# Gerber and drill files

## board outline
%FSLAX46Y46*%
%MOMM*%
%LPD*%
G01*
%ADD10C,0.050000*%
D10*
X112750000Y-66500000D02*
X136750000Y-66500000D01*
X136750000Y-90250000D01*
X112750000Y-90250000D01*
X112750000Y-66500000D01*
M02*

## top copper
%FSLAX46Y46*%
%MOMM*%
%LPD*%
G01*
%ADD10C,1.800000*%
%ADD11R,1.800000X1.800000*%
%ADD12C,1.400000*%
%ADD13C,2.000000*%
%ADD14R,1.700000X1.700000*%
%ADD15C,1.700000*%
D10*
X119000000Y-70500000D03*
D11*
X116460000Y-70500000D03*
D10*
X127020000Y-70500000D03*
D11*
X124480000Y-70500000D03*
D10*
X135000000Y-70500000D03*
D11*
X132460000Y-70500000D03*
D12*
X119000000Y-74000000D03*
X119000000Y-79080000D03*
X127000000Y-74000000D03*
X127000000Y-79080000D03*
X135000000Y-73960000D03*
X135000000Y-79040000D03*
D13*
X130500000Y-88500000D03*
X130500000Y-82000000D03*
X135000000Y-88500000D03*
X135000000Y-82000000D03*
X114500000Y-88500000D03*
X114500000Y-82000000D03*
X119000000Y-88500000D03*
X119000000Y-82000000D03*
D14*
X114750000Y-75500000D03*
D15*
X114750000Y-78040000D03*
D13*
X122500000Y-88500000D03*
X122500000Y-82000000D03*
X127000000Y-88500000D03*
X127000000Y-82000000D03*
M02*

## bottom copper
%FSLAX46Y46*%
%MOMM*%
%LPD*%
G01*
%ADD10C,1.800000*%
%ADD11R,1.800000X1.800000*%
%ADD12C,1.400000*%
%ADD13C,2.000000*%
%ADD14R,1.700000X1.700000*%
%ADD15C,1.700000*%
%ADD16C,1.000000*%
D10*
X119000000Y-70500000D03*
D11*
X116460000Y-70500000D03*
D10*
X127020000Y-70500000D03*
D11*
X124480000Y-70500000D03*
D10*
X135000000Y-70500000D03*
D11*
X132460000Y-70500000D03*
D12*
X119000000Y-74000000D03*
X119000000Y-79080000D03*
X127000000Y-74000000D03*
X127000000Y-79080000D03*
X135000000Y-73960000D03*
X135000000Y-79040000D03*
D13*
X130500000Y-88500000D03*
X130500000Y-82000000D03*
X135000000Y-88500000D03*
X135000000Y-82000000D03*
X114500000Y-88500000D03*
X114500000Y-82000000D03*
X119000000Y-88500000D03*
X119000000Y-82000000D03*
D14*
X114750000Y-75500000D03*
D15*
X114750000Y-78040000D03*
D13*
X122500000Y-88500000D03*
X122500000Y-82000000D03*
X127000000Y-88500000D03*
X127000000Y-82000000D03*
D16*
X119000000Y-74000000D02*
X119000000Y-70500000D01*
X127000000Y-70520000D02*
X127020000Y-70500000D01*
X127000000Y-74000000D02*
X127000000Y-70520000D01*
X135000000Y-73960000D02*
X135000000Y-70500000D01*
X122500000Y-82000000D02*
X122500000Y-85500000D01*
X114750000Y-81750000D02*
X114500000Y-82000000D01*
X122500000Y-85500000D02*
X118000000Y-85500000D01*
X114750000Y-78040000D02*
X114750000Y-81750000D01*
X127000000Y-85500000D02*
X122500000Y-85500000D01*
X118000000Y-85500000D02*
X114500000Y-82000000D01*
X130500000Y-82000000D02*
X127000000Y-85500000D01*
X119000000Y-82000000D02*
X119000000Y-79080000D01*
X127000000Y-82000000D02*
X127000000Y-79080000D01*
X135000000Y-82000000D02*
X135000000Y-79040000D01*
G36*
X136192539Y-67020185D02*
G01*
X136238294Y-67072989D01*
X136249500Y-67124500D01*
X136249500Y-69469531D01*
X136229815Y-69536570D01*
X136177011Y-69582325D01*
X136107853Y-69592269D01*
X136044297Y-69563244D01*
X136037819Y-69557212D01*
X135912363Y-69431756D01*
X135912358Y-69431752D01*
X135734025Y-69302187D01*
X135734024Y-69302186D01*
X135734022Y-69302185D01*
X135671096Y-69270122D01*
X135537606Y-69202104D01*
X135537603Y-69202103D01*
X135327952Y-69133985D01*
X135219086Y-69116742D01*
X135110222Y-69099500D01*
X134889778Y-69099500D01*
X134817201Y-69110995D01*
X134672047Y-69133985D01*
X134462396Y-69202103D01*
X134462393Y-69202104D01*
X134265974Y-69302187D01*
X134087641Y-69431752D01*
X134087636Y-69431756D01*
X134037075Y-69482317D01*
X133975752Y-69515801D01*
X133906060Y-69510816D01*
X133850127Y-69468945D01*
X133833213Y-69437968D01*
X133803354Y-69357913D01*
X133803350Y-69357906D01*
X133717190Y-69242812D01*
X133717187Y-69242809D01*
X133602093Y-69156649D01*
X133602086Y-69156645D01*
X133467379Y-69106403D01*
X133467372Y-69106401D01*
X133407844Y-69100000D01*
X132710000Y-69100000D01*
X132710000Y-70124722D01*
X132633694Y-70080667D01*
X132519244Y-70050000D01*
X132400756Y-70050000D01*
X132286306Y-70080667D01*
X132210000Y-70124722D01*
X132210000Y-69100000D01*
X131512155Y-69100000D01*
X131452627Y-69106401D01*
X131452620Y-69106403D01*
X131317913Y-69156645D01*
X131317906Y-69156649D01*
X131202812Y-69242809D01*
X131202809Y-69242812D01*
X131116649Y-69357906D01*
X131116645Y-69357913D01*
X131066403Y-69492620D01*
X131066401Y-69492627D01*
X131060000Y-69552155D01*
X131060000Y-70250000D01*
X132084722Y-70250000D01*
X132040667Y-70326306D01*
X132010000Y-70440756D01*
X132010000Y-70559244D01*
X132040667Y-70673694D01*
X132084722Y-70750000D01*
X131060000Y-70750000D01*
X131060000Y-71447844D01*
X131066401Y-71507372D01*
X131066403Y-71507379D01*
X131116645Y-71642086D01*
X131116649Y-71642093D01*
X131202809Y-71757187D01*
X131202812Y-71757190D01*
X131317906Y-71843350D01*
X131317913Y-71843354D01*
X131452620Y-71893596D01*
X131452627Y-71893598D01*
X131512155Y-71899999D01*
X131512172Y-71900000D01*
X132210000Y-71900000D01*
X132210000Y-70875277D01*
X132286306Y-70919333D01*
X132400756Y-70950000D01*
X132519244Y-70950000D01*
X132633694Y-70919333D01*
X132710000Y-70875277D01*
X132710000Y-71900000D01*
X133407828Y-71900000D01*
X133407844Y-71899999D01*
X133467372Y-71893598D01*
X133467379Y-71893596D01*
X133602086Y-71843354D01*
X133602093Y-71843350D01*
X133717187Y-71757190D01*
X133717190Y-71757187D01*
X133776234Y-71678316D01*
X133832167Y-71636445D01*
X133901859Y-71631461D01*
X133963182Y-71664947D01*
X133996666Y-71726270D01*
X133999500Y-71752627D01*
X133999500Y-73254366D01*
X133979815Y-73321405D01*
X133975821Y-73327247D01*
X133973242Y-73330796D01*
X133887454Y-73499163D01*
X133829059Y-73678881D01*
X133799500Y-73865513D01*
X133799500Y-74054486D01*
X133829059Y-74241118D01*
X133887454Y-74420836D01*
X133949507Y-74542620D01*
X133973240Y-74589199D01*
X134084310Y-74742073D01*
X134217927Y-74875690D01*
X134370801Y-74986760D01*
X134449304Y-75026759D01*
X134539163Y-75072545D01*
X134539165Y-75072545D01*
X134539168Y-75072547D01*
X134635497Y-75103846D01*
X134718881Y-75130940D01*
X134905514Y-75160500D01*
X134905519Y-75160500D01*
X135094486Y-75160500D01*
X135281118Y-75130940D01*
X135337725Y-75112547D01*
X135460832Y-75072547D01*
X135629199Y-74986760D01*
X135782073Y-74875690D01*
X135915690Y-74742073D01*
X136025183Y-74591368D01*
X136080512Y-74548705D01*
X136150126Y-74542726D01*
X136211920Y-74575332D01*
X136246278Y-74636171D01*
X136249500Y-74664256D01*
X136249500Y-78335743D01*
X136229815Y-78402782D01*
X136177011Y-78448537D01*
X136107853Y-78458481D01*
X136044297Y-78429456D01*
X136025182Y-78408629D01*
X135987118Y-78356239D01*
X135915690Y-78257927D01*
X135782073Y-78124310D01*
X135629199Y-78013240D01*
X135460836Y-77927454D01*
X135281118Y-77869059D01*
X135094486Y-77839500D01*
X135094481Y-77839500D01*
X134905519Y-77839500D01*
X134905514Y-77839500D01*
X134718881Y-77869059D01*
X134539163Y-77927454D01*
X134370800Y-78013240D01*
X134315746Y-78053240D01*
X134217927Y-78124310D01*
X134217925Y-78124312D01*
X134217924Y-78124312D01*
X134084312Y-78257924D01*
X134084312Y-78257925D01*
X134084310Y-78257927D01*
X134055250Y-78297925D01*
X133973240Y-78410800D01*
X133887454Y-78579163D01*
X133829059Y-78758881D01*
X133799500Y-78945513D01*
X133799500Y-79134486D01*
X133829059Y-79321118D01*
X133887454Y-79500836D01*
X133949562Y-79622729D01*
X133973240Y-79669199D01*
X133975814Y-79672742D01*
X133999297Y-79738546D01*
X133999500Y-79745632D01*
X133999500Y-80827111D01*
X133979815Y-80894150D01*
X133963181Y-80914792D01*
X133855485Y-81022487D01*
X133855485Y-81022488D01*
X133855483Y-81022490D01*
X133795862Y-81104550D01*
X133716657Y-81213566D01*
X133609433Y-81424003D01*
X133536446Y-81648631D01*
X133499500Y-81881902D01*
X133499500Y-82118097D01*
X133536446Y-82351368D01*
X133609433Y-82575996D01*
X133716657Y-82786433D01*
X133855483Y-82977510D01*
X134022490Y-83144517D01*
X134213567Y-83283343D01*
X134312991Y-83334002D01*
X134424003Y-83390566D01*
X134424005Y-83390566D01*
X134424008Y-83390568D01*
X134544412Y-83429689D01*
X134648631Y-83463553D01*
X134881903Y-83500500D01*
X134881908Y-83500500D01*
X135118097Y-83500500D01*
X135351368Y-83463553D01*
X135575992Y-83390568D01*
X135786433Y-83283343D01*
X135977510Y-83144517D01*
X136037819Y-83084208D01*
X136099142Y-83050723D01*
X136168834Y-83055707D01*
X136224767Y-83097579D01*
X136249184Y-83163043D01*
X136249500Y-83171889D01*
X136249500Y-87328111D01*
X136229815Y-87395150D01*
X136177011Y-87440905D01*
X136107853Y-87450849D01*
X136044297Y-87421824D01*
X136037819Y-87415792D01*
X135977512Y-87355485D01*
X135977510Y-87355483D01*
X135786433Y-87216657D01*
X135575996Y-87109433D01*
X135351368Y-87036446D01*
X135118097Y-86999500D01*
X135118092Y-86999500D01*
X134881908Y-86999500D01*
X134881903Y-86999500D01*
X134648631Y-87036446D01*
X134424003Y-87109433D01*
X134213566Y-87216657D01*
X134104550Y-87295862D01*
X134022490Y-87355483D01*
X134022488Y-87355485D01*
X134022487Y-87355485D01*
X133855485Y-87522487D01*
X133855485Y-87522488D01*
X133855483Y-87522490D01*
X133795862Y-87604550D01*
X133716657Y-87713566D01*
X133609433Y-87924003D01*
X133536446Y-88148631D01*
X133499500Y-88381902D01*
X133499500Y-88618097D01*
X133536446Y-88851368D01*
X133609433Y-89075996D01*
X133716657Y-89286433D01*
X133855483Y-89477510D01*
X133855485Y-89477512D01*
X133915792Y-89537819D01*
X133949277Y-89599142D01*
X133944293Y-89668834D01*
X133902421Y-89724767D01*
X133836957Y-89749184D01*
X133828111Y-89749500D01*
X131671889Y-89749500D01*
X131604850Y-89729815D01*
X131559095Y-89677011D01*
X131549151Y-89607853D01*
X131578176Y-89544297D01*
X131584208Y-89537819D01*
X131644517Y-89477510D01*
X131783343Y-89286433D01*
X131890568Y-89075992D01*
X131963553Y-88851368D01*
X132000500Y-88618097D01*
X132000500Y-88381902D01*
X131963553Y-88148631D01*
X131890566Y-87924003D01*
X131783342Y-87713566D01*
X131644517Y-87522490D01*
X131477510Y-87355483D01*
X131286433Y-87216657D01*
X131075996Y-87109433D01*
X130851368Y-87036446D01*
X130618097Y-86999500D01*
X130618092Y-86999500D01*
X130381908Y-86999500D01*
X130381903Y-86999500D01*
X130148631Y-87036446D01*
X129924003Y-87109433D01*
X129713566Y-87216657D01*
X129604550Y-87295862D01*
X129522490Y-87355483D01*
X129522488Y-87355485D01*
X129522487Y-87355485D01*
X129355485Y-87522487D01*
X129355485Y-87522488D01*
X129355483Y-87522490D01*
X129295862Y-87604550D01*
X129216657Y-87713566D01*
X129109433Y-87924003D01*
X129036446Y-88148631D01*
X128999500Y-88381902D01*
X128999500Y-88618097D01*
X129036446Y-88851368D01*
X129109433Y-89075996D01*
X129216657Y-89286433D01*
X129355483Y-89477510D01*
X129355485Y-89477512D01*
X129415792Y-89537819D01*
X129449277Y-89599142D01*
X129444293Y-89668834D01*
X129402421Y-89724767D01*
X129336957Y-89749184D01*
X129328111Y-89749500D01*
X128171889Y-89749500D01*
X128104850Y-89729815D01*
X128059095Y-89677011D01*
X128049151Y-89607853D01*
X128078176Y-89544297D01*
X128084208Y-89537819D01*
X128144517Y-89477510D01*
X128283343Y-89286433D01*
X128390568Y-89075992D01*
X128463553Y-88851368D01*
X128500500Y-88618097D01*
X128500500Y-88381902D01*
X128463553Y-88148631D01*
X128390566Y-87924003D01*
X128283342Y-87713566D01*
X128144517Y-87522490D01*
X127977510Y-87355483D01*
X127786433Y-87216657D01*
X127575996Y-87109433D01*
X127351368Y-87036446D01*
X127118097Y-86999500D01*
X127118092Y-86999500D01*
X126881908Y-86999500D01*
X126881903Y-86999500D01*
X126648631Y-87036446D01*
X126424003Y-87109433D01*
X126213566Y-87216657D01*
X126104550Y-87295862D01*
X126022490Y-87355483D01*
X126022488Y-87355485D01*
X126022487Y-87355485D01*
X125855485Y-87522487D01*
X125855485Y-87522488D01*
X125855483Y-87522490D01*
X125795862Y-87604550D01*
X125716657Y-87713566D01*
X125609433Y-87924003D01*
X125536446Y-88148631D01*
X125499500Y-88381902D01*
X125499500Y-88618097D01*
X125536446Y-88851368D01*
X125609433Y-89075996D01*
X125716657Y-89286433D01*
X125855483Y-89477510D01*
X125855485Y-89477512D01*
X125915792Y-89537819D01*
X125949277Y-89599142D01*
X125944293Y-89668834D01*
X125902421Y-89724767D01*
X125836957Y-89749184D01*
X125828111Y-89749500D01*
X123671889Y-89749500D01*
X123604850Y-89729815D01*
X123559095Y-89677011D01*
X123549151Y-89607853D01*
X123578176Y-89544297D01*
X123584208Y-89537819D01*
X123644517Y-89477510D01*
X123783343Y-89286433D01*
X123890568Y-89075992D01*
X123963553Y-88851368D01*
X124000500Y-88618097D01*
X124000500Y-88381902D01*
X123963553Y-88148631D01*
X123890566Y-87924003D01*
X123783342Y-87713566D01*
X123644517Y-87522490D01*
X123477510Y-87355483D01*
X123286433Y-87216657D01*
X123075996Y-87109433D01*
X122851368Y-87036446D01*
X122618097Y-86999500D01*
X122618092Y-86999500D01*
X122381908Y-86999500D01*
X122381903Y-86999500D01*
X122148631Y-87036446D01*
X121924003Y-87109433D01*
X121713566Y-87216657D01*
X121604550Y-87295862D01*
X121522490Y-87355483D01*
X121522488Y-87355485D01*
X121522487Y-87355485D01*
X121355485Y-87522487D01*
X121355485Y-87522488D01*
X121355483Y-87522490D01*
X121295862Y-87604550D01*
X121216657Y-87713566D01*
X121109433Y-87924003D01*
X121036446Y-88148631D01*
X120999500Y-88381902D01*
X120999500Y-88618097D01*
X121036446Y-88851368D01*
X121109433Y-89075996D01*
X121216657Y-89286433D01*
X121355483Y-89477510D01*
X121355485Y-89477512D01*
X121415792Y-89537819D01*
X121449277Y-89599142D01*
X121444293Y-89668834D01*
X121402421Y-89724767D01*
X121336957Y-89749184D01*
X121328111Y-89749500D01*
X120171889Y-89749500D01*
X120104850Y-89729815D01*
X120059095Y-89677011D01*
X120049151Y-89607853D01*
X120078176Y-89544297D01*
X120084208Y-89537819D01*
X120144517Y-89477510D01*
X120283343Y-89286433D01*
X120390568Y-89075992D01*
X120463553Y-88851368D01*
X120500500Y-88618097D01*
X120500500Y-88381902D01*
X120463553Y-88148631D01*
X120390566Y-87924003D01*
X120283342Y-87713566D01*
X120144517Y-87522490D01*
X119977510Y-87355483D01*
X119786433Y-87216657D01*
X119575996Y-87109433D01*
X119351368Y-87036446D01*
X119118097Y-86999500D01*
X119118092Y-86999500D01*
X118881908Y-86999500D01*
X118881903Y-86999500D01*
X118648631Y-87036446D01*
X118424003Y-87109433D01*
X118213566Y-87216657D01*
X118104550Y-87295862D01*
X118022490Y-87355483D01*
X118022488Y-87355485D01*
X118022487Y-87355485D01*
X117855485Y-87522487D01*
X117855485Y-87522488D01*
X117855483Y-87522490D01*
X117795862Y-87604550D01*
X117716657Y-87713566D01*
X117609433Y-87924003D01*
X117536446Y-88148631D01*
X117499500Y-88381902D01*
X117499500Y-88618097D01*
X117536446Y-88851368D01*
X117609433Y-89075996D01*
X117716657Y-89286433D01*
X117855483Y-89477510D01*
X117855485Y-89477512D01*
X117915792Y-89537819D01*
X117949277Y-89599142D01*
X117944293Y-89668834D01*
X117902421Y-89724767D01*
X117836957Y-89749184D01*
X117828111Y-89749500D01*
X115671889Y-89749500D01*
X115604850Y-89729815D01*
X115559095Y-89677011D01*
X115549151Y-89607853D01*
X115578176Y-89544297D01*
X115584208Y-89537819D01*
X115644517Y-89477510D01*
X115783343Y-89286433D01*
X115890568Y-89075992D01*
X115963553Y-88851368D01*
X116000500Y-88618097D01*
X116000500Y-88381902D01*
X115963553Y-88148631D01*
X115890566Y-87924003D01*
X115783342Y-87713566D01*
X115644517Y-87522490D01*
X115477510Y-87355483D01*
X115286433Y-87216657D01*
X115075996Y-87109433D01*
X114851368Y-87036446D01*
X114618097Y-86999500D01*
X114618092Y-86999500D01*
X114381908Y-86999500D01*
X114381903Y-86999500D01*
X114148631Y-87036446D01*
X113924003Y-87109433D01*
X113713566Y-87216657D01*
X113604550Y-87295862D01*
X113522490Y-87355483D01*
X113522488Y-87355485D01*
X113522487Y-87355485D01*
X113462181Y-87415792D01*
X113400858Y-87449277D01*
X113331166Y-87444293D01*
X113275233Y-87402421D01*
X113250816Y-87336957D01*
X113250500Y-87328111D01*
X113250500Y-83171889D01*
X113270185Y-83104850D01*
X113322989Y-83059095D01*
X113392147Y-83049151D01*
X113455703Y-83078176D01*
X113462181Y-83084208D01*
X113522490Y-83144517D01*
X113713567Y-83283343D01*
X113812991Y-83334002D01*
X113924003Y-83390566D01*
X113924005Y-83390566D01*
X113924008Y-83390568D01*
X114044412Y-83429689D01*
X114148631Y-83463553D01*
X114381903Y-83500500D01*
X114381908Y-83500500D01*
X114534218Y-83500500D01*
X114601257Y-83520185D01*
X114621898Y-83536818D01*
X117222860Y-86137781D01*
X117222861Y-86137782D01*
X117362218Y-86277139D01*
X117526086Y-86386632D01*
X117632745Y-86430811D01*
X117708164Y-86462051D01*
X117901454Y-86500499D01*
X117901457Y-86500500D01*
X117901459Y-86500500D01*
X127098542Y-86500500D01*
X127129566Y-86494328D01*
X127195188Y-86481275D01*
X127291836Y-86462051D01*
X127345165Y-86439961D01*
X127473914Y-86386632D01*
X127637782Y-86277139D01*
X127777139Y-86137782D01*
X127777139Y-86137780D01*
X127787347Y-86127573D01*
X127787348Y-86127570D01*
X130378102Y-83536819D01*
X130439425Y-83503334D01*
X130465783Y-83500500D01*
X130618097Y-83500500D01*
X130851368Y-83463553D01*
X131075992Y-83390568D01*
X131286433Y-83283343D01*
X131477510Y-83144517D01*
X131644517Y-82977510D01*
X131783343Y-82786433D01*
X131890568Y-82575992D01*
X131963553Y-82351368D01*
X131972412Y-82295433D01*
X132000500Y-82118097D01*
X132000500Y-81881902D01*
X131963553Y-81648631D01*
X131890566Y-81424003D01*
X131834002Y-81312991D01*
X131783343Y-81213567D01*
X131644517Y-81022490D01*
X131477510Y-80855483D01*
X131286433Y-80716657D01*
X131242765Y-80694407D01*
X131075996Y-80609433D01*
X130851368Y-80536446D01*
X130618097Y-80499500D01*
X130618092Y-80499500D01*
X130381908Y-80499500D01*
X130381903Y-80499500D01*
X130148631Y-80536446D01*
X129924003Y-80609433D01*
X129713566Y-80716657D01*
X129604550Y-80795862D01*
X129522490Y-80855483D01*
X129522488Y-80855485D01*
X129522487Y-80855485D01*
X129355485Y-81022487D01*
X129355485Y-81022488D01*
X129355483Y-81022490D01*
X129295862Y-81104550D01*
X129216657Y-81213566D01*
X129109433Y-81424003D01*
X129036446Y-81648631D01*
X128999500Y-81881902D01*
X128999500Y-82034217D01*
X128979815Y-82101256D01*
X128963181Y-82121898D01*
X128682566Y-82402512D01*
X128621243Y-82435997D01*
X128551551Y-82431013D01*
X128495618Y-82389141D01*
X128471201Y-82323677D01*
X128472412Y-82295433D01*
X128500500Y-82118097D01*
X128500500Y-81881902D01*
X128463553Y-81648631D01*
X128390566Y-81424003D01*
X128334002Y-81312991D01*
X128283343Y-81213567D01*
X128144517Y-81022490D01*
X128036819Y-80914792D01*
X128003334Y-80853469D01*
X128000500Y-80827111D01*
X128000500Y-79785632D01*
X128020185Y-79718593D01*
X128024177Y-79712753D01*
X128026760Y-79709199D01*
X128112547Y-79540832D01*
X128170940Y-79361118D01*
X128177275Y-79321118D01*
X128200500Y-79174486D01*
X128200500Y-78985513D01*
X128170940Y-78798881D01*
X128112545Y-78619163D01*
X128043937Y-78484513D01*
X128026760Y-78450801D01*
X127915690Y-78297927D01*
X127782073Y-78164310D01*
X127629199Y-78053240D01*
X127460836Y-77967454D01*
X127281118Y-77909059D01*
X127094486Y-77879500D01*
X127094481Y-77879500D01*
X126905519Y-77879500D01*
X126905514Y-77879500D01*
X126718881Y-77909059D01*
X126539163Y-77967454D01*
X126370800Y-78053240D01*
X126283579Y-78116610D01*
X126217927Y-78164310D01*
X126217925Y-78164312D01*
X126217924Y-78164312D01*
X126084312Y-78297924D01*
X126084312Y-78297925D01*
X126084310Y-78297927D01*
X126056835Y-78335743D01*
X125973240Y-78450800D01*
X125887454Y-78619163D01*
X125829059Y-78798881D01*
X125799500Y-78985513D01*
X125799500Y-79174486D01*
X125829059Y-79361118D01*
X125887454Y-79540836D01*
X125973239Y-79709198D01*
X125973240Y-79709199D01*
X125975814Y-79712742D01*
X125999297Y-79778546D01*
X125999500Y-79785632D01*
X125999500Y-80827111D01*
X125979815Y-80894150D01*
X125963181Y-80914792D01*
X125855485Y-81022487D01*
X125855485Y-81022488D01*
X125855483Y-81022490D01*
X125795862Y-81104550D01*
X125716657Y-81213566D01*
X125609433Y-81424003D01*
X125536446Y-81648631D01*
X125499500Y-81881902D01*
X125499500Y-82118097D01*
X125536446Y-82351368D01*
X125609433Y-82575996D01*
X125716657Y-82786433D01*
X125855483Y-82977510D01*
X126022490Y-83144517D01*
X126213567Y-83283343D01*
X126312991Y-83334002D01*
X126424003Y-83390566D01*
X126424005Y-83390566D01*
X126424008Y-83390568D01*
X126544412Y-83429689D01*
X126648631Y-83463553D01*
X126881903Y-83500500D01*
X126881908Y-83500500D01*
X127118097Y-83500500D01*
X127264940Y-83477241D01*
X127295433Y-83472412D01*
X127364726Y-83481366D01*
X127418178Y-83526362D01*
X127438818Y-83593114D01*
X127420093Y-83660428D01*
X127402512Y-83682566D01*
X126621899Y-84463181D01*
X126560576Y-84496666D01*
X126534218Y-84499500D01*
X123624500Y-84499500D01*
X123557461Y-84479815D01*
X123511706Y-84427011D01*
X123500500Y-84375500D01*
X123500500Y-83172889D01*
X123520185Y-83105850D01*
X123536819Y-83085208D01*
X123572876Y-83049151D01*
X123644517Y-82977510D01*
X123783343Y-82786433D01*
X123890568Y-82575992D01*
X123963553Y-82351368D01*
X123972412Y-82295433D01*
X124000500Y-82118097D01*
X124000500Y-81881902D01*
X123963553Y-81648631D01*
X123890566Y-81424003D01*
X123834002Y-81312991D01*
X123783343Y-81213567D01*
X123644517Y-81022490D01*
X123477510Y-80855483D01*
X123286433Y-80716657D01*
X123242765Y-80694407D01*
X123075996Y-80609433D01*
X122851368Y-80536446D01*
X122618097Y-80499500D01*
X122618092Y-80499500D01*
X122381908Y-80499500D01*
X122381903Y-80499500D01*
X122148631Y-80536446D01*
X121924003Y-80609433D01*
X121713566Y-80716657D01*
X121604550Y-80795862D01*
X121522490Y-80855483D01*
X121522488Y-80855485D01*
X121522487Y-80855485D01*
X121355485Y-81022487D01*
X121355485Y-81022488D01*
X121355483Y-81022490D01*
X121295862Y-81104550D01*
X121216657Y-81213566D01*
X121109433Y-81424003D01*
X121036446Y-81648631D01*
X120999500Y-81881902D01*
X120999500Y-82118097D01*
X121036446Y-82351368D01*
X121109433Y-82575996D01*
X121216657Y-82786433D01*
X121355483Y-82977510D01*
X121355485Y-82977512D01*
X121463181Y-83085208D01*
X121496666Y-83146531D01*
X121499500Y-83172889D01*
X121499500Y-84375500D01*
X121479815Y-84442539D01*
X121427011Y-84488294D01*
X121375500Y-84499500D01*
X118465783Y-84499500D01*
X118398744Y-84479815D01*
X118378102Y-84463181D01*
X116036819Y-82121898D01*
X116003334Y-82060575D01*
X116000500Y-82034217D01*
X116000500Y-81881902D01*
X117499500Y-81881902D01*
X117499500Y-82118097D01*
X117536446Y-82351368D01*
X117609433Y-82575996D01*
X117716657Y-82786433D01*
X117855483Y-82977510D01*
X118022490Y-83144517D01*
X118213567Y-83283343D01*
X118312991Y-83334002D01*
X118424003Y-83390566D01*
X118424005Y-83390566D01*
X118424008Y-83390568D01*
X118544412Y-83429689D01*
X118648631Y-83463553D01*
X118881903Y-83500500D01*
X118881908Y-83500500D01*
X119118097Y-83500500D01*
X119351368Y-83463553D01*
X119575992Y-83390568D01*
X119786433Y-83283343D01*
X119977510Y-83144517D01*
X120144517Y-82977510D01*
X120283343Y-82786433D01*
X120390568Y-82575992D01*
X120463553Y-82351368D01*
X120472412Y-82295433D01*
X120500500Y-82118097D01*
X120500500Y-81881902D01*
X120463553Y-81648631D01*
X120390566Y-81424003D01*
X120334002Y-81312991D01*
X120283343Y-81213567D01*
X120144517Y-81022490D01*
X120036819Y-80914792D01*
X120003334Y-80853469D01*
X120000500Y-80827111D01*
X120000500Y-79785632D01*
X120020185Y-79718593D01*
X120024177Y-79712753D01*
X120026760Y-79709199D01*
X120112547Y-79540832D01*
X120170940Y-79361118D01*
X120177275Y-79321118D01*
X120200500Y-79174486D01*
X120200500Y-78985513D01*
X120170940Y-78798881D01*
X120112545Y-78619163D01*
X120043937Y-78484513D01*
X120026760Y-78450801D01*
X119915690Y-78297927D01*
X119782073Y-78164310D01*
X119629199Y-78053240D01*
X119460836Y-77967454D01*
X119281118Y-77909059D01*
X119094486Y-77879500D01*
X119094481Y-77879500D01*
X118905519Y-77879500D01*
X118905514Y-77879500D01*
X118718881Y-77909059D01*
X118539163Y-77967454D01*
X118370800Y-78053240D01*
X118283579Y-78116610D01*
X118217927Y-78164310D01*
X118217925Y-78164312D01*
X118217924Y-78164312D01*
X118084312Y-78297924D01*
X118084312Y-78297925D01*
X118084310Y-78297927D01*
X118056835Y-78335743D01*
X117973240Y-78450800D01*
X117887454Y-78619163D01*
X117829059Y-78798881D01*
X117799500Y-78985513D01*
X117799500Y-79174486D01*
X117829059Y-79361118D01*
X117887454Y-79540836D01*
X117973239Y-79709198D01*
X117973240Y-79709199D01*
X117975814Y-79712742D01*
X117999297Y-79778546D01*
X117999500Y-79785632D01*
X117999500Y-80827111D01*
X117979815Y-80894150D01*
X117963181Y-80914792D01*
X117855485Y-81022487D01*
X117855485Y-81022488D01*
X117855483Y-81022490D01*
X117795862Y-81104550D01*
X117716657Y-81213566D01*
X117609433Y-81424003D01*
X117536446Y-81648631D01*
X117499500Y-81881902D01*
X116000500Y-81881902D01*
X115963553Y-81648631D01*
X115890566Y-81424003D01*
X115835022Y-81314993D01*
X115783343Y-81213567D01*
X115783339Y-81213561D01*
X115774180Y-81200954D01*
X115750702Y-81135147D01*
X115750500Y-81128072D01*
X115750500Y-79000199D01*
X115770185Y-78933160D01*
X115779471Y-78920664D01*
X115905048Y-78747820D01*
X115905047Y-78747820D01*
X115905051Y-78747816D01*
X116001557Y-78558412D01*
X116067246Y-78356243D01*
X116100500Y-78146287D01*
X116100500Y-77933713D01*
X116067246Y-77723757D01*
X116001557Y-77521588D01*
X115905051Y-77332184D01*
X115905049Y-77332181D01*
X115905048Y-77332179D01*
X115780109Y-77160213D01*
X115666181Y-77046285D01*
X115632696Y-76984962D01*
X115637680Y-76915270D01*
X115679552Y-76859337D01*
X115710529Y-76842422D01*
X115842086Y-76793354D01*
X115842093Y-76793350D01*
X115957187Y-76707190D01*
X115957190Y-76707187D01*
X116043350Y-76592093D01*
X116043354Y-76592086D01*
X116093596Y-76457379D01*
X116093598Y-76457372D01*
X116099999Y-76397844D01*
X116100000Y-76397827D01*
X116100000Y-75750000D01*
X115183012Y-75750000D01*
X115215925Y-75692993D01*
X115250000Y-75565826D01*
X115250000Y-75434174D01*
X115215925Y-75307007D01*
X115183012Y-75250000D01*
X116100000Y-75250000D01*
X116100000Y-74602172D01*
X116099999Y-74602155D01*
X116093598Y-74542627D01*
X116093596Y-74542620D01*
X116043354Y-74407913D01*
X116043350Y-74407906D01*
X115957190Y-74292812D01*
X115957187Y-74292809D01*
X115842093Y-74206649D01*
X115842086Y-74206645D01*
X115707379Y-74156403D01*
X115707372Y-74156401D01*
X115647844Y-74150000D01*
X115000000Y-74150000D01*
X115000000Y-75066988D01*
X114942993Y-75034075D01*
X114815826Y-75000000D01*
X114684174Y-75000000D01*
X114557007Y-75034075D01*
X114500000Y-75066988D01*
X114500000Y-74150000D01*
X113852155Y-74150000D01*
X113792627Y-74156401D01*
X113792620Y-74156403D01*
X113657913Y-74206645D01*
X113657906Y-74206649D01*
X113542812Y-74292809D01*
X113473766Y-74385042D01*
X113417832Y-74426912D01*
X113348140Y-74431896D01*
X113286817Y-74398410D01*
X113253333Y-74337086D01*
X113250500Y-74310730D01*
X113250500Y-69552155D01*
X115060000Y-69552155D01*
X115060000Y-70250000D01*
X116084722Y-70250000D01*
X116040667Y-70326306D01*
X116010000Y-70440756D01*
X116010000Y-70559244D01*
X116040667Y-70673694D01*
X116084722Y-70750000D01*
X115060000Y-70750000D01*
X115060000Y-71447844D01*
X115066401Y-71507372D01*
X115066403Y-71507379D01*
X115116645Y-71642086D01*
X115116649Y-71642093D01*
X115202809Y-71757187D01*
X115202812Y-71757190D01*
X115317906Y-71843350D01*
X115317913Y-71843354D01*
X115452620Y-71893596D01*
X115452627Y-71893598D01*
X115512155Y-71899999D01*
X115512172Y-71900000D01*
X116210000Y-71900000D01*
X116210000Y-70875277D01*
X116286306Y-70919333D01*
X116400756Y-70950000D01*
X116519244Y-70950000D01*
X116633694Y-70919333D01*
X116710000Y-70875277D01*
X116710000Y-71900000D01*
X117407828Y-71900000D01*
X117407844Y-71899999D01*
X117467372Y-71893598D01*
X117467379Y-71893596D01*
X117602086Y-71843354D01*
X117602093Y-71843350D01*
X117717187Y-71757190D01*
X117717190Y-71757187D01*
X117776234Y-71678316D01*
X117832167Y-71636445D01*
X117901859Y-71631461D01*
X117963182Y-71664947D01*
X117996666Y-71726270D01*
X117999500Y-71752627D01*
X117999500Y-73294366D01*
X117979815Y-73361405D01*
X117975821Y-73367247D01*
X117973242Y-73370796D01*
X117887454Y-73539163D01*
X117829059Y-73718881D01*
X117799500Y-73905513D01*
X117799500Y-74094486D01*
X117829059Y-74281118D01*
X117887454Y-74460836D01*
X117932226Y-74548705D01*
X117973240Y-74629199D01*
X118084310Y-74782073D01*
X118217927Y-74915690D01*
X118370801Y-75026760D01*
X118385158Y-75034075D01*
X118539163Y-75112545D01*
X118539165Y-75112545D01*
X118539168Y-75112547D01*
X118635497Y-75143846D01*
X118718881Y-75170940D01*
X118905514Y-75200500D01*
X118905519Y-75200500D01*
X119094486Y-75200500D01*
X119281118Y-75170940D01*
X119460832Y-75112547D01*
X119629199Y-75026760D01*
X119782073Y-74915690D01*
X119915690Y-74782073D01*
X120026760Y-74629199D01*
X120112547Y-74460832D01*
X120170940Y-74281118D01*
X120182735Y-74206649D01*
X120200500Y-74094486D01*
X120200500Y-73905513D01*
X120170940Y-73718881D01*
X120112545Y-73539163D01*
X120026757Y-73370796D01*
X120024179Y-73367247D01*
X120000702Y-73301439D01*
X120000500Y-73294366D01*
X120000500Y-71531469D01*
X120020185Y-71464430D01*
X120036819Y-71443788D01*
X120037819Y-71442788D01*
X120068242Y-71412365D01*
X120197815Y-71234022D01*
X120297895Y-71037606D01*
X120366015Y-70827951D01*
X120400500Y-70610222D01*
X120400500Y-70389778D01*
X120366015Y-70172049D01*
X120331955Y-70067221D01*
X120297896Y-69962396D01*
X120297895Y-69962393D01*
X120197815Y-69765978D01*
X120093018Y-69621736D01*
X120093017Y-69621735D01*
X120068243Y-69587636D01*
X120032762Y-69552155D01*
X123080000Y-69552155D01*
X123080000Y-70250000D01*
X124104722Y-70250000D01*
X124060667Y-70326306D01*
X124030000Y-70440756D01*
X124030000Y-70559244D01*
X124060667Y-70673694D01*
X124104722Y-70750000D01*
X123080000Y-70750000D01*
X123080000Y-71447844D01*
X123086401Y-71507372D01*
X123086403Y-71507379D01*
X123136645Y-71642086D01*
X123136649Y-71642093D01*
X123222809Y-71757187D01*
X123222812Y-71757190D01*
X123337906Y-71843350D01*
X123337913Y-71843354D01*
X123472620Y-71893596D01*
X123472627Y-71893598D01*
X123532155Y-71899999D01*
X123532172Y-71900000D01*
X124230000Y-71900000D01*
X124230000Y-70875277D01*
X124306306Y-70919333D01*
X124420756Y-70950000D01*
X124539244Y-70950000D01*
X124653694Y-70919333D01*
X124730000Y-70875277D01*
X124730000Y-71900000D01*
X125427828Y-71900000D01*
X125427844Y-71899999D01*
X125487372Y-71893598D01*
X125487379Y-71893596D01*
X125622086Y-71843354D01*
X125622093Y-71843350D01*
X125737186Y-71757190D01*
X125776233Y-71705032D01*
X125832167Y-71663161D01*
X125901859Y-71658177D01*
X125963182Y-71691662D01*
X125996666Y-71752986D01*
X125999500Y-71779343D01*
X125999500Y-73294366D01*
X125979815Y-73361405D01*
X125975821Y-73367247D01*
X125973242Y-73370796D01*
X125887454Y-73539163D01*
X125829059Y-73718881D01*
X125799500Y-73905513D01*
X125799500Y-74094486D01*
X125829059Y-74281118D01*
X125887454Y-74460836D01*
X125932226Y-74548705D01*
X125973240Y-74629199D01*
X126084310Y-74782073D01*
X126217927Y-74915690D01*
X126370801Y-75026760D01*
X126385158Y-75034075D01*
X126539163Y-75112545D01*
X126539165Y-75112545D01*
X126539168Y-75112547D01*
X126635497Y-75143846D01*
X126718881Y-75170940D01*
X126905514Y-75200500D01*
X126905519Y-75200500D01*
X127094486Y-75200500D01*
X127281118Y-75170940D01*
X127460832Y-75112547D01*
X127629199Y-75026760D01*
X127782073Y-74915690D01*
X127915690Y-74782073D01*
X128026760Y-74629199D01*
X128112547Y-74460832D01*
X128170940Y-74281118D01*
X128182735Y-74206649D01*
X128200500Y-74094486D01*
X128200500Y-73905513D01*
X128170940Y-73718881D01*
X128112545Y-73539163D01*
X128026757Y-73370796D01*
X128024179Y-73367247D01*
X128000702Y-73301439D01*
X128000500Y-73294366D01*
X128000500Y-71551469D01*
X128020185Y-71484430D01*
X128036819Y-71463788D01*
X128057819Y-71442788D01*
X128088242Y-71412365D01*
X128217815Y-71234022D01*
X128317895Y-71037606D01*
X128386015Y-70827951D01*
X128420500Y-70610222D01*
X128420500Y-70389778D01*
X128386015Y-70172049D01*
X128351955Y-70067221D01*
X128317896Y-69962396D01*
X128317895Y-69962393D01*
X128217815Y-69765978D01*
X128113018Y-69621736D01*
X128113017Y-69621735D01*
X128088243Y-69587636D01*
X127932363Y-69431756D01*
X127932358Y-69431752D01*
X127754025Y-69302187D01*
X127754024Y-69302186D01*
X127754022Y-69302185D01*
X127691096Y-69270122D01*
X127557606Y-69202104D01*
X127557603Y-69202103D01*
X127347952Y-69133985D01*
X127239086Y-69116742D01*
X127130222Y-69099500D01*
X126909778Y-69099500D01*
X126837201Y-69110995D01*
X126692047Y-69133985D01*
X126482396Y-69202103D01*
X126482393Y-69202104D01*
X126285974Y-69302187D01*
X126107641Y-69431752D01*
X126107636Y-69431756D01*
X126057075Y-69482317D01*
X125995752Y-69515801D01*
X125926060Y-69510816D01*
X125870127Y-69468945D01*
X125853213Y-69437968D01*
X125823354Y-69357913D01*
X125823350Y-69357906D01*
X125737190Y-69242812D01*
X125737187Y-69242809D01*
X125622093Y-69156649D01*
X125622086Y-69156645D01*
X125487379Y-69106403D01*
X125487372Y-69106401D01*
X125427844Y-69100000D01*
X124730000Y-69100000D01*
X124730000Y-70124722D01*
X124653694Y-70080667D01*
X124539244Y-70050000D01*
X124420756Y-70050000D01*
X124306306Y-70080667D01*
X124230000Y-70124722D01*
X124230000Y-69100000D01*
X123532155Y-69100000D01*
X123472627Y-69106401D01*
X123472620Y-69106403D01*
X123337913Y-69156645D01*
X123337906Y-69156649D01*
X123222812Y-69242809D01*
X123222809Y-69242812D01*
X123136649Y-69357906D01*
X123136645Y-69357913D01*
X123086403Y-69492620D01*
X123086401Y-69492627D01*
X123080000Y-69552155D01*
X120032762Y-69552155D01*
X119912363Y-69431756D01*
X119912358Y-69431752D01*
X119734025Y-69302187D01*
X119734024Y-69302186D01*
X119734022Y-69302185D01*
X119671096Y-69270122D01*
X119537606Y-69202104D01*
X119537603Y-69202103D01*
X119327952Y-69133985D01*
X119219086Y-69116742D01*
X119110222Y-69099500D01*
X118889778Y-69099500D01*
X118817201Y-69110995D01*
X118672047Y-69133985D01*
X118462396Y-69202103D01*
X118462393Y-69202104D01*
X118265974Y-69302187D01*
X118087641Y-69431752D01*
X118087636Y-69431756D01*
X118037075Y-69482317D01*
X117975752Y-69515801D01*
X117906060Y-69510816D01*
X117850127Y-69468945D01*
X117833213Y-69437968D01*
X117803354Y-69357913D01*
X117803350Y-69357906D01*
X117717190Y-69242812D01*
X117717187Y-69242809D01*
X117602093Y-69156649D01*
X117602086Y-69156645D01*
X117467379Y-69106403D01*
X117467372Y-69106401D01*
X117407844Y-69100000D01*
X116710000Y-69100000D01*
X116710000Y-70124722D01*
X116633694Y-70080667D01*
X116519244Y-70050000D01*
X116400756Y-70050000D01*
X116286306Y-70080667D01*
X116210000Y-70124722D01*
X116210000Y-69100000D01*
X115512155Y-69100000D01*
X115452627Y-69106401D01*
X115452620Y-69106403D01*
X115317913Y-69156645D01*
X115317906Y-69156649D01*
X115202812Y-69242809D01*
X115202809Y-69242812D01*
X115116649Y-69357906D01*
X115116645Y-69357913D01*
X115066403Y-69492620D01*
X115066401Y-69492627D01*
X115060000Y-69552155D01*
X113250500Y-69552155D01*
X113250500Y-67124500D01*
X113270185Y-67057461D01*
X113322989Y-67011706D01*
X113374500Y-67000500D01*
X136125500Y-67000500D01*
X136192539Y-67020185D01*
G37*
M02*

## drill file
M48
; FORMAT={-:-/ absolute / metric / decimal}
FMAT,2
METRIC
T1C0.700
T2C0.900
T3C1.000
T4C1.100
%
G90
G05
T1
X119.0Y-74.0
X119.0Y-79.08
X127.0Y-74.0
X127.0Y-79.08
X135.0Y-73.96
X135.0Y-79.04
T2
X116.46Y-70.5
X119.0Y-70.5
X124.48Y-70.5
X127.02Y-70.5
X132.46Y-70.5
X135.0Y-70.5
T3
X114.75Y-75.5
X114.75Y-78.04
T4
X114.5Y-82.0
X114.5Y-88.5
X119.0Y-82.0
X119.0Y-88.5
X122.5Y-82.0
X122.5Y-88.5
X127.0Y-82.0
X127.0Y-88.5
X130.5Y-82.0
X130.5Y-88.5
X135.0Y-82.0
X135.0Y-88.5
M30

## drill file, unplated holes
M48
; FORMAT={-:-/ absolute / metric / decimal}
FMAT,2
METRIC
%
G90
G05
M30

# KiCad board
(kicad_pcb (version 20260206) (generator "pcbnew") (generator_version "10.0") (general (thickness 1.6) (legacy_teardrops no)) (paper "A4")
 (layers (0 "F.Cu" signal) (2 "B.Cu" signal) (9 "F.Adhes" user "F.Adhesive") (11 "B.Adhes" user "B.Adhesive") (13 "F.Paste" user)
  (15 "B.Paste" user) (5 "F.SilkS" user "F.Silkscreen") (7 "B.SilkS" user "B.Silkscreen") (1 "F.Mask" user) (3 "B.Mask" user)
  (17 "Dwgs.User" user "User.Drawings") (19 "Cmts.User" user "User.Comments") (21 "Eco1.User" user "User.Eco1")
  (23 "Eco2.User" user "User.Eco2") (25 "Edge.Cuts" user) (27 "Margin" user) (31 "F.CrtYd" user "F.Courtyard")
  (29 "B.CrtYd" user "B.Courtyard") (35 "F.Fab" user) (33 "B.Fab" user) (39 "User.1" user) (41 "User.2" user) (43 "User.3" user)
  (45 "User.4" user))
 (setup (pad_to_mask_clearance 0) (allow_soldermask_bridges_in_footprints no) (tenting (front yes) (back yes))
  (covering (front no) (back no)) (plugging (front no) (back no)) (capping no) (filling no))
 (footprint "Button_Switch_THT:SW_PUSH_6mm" (layer "F.Cu") (at 130.5 88.5 90)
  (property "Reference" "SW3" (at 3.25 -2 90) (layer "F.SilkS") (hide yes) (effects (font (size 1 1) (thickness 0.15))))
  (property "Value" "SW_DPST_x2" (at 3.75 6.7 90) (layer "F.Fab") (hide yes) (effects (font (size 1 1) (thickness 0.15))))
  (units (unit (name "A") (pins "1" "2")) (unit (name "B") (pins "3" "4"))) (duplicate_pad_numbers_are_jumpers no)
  (pad "1" thru_hole circle (at 0 0 180) (size 2 2) (drill 1.1) (layers "*.Cu" "*.Mask") (remove_unused_layers no) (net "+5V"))
  (pad "1" thru_hole circle (at 6.5 0 180) (size 2 2) (drill 1.1) (layers "*.Cu" "*.Mask") (remove_unused_layers no) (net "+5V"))
  (pad "2" thru_hole circle (at 0 4.5 180) (size 2 2) (drill 1.1) (layers "*.Cu" "*.Mask") (remove_unused_layers no) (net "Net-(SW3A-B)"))
  (pad "2" thru_hole circle (at 6.5 4.5 180) (size 2 2) (drill 1.1) (layers "*.Cu" "*.Mask") (remove_unused_layers no) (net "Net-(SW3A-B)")))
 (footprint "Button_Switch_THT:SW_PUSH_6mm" (layer "F.Cu") (at 114.5 88.5 90)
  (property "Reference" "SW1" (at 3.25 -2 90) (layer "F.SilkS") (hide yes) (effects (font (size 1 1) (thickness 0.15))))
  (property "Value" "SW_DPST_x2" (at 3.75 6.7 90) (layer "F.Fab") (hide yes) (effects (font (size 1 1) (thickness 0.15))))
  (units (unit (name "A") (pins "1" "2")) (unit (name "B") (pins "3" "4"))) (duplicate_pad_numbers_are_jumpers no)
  (pad "1" thru_hole circle (at 0 0 180) (size 2 2) (drill 1.1) (layers "*.Cu" "*.Mask") (remove_unused_layers no) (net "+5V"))
  (pad "1" thru_hole circle (at 6.5 0 180) (size 2 2) (drill 1.1) (layers "*.Cu" "*.Mask") (remove_unused_layers no) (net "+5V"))
  (pad "2" thru_hole circle (at 0 4.5 180) (size 2 2) (drill 1.1) (layers "*.Cu" "*.Mask") (remove_unused_layers no) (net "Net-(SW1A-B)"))
  (pad "2" thru_hole circle (at 6.5 4.5 180) (size 2 2) (drill 1.1) (layers "*.Cu" "*.Mask") (remove_unused_layers no) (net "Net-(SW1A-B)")))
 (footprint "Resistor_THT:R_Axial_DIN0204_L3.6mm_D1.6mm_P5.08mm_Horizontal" (layer "F.Cu") (at 127 79.08 90)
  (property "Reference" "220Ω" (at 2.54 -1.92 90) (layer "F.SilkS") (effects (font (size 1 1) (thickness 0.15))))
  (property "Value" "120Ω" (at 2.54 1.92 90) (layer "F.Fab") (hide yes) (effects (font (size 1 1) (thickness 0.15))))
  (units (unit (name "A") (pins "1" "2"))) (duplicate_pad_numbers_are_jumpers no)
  (pad "1" thru_hole circle (at 0 0 90) (size 1.4 1.4) (drill 0.7) (layers "*.Cu" "*.Mask") (remove_unused_layers no) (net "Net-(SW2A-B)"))
  (pad "2" thru_hole circle (at 5.08 0 90) (size 1.4 1.4) (drill 0.7) (layers "*.Cu" "*.Mask") (remove_unused_layers no) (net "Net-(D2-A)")))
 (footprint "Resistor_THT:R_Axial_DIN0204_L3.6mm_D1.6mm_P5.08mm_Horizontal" (layer "F.Cu") (at 135 79.04 90)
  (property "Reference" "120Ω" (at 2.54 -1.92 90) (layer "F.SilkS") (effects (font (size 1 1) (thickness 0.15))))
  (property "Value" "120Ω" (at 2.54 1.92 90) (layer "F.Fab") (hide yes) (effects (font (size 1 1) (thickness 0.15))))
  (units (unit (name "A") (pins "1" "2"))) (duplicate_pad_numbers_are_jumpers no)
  (pad "1" thru_hole circle (at 0 0 90) (size 1.4 1.4) (drill 0.7) (layers "*.Cu" "*.Mask") (remove_unused_layers no) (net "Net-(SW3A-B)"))
  (pad "2" thru_hole circle (at 5.08 0 90) (size 1.4 1.4) (drill 0.7) (layers "*.Cu" "*.Mask") (remove_unused_layers no) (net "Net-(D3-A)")))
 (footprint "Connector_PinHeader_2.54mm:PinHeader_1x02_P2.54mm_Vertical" (layer "F.Cu") (at 114.75 75.5)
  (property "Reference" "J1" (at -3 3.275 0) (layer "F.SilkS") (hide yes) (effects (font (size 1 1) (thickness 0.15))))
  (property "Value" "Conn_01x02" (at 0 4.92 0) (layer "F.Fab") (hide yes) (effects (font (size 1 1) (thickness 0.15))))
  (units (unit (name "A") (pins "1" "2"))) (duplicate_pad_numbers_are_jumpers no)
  (pad "1" thru_hole rect (at 0 0) (size 1.7 1.7) (drill 1) (layers "*.Cu" "*.Mask") (remove_unused_layers no) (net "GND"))
  (pad "2" thru_hole circle (at 0 2.54) (size 1.7 1.7) (drill 1) (layers "*.Cu" "*.Mask") (remove_unused_layers no) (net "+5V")))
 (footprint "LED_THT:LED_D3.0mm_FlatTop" (layer "F.Cu") (at 132.46 70.5)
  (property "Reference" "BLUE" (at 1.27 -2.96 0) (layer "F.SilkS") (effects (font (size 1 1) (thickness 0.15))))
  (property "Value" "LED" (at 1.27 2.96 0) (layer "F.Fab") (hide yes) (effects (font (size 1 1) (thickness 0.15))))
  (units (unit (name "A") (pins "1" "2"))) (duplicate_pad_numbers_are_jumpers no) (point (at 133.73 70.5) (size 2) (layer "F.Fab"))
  (pad "1" thru_hole rect (at 0 0) (size 1.8 1.8) (drill 0.9) (layers "*.Cu" "*.Mask") (remove_unused_layers no) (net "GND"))
  (pad "2" thru_hole circle (at 2.54 0) (size 1.8 1.8) (drill 0.9) (layers "*.Cu" "*.Mask") (remove_unused_layers no) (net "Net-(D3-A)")))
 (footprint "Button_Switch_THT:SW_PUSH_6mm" (layer "F.Cu") (at 122.5 88.5 90)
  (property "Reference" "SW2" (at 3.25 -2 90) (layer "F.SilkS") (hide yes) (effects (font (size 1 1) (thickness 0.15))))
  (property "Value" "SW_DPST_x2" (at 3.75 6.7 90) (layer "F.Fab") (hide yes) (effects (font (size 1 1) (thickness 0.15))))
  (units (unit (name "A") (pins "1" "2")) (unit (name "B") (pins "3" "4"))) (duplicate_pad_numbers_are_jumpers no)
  (pad "1" thru_hole circle (at 0 0 180) (size 2 2) (drill 1.1) (layers "*.Cu" "*.Mask") (remove_unused_layers no) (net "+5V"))
  (pad "1" thru_hole circle (at 6.5 0 180) (size 2 2) (drill 1.1) (layers "*.Cu" "*.Mask") (remove_unused_layers no) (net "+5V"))
  (pad "2" thru_hole circle (at 0 4.5 180) (size 2 2) (drill 1.1) (layers "*.Cu" "*.Mask") (remove_unused_layers no) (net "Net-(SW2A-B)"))
  (pad "2" thru_hole circle (at 6.5 4.5 180) (size 2 2) (drill 1.1) (layers "*.Cu" "*.Mask") (remove_unused_layers no) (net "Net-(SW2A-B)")))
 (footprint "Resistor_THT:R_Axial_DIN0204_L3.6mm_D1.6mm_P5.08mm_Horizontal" (layer "F.Cu") (at 119 79.08 90)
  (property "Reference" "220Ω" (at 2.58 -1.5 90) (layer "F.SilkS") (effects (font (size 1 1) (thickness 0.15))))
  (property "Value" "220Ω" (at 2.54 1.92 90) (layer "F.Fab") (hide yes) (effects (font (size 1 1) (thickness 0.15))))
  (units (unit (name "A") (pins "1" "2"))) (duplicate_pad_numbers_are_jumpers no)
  (pad "1" thru_hole circle (at 0 0 90) (size 1.4 1.4) (drill 0.7) (layers "*.Cu" "*.Mask") (remove_unused_layers no) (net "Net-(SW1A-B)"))
  (pad "2" thru_hole circle (at 5.08 0 90) (size 1.4 1.4) (drill 0.7) (layers "*.Cu" "*.Mask") (remove_unused_layers no) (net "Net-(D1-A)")))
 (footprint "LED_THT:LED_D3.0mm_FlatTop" (layer "F.Cu") (at 124.48 70.5)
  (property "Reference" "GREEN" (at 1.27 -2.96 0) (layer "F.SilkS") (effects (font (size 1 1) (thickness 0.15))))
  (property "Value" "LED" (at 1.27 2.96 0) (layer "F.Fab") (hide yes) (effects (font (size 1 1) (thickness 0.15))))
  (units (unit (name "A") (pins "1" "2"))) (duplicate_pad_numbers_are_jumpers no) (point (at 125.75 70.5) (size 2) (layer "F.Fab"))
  (pad "1" thru_hole rect (at 0 0) (size 1.8 1.8) (drill 0.9) (layers "*.Cu" "*.Mask") (remove_unused_layers no) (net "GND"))
  (pad "2" thru_hole circle (at 2.54 0) (size 1.8 1.8) (drill 0.9) (layers "*.Cu" "*.Mask") (remove_unused_layers no) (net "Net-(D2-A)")))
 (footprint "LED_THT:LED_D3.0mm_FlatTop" (layer "F.Cu") (at 116.46 70.5)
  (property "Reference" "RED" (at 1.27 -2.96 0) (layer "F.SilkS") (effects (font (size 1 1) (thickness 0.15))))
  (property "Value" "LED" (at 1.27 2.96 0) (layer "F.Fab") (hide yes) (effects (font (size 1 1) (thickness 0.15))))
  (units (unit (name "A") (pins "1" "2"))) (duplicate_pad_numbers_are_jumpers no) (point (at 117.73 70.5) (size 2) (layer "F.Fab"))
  (pad "1" thru_hole rect (at 0 0) (size 1.8 1.8) (drill 0.9) (layers "*.Cu" "*.Mask") (remove_unused_layers no) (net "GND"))
  (pad "2" thru_hole circle (at 2.54 0) (size 1.8 1.8) (drill 0.9) (layers "*.Cu" "*.Mask") (remove_unused_layers no) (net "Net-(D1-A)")))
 (gr_rect (start 112.75 66.5) (end 136.75 90.25) (stroke (width 0.05) (type default)) (fill no) (layer "Edge.Cuts"))
 (segment (start 122.5 82) (end 122.5 85.5) (width 1) (layer "B.Cu") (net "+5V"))
 (segment (start 114.75 81.75) (end 114.5 82) (width 1) (layer "B.Cu") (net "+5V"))
 (segment (start 122.5 85.5) (end 118 85.5) (width 1) (layer "B.Cu") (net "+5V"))
 (segment (start 114.75 78.04) (end 114.75 81.75) (width 1) (layer "B.Cu") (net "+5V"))
 (segment (start 127 85.5) (end 122.5 85.5) (width 1) (layer "B.Cu") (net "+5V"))
 (segment (start 118 85.5) (end 114.5 82) (width 1) (layer "B.Cu") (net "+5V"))
 (segment (start 130.5 82) (end 127 85.5) (width 1) (layer "B.Cu") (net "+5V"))
 (segment (start 135 82) (end 135 79.04) (width 1) (layer "B.Cu") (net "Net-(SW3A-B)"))
 (segment (start 119 82) (end 119 79.08) (width 1) (layer "B.Cu") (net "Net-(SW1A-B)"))
 (segment (start 127 82) (end 127 79.08) (width 1) (layer "B.Cu") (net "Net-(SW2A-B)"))
 (segment (start 127 70.52) (end 127.02 70.5) (width 1) (layer "B.Cu") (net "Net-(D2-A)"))
 (segment (start 127 74) (end 127 70.52) (width 1) (layer "B.Cu") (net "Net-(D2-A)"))
 (segment (start 135 73.96) (end 135 70.5) (width 1) (layer "B.Cu") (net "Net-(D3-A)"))
 (segment (start 119 74) (end 119 70.5) (width 1) (layer "B.Cu") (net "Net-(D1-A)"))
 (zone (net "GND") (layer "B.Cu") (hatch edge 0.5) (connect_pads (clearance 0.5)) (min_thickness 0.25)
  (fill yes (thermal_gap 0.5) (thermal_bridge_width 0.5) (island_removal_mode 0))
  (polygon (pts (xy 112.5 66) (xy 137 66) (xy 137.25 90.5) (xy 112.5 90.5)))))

